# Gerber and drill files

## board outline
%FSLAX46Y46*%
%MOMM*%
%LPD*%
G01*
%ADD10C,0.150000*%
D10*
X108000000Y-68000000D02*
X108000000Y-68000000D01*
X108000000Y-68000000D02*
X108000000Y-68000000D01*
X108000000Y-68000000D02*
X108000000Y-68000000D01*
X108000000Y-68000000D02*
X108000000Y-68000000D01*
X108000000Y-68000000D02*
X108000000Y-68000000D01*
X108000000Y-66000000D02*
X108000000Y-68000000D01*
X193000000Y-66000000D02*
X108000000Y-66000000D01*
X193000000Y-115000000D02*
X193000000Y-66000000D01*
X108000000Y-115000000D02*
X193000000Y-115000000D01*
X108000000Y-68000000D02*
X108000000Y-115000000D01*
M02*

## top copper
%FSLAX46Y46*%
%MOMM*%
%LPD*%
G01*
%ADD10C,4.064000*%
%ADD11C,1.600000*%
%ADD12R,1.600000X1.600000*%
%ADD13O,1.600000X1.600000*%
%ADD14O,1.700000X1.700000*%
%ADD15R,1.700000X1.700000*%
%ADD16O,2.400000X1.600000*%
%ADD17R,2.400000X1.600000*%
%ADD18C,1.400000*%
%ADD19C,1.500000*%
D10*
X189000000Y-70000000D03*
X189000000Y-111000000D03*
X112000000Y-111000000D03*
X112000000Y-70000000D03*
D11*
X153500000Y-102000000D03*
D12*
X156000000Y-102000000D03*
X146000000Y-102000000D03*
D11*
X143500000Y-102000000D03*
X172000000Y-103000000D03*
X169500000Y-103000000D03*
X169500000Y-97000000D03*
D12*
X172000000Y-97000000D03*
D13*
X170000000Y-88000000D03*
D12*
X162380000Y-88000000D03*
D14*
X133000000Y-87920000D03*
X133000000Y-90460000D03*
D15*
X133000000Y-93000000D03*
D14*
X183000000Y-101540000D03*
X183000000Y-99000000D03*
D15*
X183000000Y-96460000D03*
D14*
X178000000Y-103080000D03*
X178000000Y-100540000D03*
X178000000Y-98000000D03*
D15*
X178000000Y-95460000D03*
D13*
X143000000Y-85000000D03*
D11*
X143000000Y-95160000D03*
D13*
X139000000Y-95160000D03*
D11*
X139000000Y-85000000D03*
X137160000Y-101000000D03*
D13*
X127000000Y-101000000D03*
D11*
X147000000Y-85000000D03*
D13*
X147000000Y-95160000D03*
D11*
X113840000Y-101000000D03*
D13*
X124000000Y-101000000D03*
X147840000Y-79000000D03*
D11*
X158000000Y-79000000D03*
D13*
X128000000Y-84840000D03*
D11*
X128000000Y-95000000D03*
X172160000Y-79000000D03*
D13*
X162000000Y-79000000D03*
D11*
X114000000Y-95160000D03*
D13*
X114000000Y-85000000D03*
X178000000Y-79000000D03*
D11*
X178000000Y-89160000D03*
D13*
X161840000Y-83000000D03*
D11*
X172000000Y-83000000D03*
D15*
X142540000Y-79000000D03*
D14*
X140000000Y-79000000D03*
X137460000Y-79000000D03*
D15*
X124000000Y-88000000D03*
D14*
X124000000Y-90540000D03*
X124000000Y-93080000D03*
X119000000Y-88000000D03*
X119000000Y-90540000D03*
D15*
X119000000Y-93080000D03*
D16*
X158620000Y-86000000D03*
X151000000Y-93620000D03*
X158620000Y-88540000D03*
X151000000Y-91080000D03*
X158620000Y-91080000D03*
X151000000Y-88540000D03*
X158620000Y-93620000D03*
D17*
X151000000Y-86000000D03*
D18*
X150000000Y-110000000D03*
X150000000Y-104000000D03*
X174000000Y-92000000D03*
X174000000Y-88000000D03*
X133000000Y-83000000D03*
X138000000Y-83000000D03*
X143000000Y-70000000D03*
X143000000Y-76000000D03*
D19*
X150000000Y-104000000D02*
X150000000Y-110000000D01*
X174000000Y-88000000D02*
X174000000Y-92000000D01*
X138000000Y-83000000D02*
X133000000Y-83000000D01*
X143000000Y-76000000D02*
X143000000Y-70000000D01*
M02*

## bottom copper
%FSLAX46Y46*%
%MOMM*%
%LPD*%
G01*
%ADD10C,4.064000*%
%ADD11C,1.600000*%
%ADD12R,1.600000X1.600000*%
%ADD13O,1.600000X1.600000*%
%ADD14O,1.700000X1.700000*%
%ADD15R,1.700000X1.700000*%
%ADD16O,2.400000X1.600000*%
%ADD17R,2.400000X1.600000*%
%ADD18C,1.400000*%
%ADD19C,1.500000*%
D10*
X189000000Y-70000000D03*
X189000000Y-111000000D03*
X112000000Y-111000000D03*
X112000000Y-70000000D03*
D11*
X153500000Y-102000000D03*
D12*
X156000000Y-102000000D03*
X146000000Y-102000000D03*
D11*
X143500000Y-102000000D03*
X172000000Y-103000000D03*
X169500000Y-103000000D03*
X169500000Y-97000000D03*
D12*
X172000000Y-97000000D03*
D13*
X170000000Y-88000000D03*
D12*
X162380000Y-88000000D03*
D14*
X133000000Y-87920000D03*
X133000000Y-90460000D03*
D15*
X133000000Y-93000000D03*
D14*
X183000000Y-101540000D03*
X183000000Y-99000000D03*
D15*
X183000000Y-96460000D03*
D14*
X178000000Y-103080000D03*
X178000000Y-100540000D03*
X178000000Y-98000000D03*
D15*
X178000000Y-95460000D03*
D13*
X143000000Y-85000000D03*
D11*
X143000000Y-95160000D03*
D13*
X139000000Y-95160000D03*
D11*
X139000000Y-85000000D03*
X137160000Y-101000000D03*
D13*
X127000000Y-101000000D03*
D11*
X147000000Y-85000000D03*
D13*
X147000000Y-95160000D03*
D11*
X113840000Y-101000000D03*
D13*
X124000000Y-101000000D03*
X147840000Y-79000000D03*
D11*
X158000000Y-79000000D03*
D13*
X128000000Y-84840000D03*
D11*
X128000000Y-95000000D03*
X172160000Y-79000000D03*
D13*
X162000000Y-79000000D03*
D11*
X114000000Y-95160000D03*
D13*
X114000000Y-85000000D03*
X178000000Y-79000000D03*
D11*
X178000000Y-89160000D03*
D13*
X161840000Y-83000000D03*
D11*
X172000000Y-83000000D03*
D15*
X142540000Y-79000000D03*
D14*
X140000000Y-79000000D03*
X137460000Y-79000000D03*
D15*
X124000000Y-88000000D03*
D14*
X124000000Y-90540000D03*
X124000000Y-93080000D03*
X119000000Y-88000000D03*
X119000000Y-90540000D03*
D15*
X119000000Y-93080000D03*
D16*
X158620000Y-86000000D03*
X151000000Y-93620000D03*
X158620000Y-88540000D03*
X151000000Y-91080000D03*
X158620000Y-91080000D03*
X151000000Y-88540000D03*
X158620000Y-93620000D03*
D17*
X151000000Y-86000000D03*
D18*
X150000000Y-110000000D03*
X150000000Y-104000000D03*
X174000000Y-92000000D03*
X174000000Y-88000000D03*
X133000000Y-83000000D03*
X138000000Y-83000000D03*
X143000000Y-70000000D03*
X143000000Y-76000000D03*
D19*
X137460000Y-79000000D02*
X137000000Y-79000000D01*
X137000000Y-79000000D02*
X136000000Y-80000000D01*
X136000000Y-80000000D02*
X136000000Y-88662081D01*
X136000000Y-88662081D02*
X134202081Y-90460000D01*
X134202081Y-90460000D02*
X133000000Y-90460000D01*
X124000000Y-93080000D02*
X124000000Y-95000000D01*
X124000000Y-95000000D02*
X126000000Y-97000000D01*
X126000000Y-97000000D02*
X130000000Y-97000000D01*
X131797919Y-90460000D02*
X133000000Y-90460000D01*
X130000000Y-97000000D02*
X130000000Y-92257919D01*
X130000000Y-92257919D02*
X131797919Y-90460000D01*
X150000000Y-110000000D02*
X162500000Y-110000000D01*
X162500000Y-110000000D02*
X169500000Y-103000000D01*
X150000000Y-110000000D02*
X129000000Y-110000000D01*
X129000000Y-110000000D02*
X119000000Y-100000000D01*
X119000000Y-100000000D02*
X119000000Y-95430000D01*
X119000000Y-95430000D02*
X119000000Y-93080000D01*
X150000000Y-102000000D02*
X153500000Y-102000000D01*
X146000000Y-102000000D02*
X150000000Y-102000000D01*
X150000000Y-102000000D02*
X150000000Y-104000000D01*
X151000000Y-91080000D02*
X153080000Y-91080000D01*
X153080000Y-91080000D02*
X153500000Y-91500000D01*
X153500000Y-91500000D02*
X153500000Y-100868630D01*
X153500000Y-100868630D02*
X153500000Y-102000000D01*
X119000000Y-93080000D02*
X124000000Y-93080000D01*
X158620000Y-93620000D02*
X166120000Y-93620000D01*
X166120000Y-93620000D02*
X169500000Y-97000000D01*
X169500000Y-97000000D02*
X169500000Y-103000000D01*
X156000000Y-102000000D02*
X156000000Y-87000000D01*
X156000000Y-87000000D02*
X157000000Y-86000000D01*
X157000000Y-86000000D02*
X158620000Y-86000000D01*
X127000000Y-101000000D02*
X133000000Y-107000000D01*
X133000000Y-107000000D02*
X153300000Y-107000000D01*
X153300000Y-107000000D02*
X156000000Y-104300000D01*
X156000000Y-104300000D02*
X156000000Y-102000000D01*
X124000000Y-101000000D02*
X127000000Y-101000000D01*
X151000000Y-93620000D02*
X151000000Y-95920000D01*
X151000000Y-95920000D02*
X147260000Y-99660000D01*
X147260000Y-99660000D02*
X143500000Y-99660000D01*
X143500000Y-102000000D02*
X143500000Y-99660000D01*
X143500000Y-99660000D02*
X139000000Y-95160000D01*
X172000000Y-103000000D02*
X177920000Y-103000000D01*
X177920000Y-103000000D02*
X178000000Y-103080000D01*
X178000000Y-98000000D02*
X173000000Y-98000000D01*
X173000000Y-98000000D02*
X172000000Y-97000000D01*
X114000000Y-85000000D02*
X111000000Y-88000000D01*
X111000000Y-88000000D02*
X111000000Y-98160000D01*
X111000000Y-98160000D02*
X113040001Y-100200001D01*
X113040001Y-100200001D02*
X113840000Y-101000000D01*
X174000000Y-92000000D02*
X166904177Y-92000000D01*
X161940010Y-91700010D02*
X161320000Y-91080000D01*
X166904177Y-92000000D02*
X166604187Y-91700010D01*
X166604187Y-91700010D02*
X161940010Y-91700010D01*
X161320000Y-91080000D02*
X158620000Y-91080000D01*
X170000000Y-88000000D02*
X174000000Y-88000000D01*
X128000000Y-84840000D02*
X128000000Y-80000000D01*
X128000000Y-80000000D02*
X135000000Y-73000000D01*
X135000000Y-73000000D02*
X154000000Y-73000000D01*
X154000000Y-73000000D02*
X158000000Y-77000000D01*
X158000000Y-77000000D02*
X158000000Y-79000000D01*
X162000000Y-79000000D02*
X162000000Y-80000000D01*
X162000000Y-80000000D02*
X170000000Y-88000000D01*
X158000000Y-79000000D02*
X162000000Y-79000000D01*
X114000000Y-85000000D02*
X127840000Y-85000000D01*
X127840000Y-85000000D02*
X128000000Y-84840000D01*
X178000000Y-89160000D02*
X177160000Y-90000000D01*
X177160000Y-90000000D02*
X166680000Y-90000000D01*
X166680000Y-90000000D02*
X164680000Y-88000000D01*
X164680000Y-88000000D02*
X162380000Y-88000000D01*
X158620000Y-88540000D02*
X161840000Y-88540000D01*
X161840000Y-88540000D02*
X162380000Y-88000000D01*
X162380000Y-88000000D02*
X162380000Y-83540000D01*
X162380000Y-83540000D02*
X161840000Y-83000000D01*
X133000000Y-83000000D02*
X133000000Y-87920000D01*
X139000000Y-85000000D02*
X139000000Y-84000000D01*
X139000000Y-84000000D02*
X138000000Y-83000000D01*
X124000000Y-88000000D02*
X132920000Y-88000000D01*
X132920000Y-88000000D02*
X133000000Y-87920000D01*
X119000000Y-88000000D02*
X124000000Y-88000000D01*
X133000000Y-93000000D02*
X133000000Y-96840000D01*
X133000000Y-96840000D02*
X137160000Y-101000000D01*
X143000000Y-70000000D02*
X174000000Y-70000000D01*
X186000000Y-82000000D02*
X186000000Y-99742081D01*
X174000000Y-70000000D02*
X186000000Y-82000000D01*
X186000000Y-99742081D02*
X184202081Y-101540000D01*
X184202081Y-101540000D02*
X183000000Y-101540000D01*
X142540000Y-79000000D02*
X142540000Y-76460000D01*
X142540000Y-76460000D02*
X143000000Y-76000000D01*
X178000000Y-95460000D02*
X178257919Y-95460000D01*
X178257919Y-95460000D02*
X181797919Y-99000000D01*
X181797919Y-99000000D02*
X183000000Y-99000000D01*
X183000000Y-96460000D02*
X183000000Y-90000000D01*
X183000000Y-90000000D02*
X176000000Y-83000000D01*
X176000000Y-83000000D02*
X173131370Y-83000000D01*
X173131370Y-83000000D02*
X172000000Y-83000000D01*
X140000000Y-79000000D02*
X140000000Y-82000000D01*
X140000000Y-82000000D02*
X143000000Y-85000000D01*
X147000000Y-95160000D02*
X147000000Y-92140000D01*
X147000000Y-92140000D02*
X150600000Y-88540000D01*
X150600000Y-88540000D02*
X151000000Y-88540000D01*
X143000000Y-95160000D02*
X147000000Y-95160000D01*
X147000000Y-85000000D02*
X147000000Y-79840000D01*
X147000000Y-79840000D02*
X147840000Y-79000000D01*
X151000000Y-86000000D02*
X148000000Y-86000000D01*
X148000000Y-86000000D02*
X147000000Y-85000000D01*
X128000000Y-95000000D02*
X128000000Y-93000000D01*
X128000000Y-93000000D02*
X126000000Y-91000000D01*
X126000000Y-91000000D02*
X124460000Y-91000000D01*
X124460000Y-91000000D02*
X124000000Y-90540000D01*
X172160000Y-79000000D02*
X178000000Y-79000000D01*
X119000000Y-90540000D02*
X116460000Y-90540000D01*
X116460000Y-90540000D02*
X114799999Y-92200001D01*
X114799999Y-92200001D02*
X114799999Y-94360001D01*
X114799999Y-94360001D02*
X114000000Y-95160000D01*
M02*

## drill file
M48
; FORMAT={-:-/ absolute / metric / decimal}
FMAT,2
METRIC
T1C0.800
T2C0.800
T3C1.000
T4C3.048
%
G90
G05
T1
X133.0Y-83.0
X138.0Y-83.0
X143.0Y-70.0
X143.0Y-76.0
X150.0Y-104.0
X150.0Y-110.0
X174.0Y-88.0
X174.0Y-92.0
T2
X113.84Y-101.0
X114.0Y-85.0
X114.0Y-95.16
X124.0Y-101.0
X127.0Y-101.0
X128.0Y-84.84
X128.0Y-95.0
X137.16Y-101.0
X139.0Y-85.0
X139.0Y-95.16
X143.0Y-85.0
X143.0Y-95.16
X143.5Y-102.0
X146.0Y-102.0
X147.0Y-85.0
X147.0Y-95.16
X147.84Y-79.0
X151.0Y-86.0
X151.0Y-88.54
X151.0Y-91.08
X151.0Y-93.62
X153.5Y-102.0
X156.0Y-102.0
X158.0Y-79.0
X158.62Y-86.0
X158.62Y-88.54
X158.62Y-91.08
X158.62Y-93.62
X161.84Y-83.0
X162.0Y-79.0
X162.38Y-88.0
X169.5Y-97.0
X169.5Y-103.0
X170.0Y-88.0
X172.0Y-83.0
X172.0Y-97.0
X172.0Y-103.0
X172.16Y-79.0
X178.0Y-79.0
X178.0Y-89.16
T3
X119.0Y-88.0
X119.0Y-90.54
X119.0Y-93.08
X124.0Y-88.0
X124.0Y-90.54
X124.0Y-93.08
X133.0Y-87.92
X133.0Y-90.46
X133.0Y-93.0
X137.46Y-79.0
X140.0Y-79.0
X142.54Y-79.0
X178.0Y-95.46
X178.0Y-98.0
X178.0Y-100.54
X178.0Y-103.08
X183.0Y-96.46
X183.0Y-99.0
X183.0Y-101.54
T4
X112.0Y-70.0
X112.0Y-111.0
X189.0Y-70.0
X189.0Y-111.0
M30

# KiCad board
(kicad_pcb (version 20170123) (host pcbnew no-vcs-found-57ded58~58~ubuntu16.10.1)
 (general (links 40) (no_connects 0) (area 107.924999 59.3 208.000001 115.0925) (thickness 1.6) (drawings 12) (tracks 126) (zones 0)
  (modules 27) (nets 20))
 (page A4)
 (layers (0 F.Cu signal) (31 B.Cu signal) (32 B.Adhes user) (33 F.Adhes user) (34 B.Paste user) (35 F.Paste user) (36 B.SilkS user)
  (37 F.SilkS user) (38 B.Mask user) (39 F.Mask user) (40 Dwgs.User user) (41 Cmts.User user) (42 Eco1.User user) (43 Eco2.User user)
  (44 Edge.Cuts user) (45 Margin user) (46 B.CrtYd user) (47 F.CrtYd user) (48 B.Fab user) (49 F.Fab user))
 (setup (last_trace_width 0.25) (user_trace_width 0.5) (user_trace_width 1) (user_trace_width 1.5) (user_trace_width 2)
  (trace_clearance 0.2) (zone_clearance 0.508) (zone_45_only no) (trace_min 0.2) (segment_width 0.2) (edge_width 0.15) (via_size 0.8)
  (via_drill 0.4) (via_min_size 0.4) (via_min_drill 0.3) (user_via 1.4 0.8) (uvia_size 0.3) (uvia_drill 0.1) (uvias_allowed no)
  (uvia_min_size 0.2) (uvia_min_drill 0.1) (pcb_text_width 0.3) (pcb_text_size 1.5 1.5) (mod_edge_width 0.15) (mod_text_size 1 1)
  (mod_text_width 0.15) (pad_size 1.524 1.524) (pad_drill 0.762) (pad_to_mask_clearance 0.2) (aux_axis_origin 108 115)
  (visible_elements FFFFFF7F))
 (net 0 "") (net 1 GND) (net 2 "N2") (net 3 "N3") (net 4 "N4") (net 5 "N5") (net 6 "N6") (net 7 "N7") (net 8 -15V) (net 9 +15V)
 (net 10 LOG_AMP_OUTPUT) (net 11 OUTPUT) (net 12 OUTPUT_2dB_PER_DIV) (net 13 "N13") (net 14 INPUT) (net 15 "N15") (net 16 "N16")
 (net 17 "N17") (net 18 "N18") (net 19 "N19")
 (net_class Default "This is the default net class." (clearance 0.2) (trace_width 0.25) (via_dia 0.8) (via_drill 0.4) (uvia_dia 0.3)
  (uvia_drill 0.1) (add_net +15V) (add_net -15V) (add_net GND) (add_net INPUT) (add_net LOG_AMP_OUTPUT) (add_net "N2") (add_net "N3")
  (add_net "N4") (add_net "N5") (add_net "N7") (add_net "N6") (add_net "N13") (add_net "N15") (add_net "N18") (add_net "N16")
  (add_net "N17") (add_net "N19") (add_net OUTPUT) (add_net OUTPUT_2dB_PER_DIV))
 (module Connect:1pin (layer F.Cu) (at 189 70)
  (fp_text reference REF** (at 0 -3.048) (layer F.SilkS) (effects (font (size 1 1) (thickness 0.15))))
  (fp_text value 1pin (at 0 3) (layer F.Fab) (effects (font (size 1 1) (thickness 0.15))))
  (pad 1 thru_hole circle (at 0 0) (size 4.064 4.064) (drill 3.048) (layers *.Cu *.Mask)))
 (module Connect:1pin (layer F.Cu) (at 189 111)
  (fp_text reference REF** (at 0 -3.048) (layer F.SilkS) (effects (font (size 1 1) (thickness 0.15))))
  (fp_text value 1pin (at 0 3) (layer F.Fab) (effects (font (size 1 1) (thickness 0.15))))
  (pad 1 thru_hole circle (at 0 0) (size 4.064 4.064) (drill 3.048) (layers *.Cu *.Mask)))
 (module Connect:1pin (layer F.Cu) (at 112 111)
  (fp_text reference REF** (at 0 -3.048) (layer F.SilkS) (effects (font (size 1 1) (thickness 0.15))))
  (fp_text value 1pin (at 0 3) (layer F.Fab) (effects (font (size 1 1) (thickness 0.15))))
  (pad 1 thru_hole circle (at 0 0) (size 4.064 4.064) (drill 3.048) (layers *.Cu *.Mask)))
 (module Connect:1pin (layer F.Cu) (at 112 70)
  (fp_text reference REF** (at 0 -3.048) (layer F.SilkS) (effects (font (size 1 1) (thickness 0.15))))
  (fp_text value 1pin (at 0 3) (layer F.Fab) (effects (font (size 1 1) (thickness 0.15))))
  (pad 1 thru_hole circle (at 0 0) (size 4.064 4.064) (drill 3.048) (layers *.Cu *.Mask)))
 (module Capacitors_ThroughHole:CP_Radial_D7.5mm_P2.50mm (layer F.Cu) (at 156 102 180)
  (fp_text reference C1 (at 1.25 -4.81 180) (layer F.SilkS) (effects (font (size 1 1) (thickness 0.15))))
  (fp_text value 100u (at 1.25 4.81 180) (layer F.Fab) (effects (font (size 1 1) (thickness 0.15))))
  (pad 2 thru_hole circle (at 2.5 0 180) (size 1.6 1.6) (drill 0.8) (layers *.Cu *.Mask) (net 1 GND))
  (pad 1 thru_hole rect (at 0 0 180) (size 1.6 1.6) (drill 0.8) (layers *.Cu *.Mask) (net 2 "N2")))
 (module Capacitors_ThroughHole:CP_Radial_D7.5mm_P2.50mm (layer F.Cu) (at 146 102 180)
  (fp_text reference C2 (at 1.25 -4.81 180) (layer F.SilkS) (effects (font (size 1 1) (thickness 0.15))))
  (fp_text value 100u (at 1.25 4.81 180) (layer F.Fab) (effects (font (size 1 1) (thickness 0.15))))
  (pad 1 thru_hole rect (at 0 0 180) (size 1.6 1.6) (drill 0.8) (layers *.Cu *.Mask) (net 1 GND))
  (pad 2 thru_hole circle (at 2.5 0 180) (size 1.6 1.6) (drill 0.8) (layers *.Cu *.Mask) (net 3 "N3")))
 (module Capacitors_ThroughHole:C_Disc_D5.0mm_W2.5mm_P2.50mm (layer F.Cu) (at 169.5 103)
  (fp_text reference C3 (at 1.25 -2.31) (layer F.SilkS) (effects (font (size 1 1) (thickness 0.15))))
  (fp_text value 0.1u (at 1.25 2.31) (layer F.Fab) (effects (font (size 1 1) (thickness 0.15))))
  (pad 2 thru_hole circle (at 2.5 0) (size 1.6 1.6) (drill 0.8) (layers *.Cu *.Mask) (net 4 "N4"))
  (pad 1 thru_hole circle (at 0 0) (size 1.6 1.6) (drill 0.8) (layers *.Cu *.Mask) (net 1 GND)))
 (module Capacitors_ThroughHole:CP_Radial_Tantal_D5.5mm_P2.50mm (layer F.Cu) (at 172 97 180)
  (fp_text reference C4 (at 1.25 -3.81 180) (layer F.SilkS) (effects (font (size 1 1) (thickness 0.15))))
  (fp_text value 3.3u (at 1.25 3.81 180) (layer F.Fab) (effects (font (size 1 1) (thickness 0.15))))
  (pad 2 thru_hole circle (at 2.5 0 180) (size 1.6 1.6) (drill 0.8) (layers *.Cu *.Mask) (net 1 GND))
  (pad 1 thru_hole rect (at 0 0 180) (size 1.6 1.6) (drill 0.8) (layers *.Cu *.Mask) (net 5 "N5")))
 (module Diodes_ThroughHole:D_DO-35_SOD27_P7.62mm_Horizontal (layer F.Cu) (at 162.38 88)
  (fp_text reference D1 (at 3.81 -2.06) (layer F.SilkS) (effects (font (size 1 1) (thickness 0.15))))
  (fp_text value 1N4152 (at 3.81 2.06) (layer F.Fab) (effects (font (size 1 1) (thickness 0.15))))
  (pad 2 thru_hole oval (at 7.62 0) (size 1.6 1.6) (drill 0.8) (layers *.Cu *.Mask) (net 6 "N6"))
  (pad 1 thru_hole rect (at 0 0) (size 1.6 1.6) (drill 0.8) (layers *.Cu *.Mask) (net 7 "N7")))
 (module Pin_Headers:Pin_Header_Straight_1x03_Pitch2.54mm (layer F.Cu) (at 133 93 180)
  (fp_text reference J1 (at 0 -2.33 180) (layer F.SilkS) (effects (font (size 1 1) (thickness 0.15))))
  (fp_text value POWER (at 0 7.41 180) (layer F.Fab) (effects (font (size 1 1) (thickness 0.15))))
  (pad 3 thru_hole oval (at 0 5.08 180) (size 1.7 1.7) (drill 1) (layers *.Cu *.Mask) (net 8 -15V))
  (pad 2 thru_hole oval (at 0 2.54 180) (size 1.7 1.7) (drill 1) (layers *.Cu *.Mask) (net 1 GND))
  (pad 1 thru_hole rect (at 0 0 180) (size 1.7 1.7) (drill 1) (layers *.Cu *.Mask) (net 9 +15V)))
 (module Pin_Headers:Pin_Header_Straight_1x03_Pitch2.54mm (layer F.Cu) (at 183 96.46)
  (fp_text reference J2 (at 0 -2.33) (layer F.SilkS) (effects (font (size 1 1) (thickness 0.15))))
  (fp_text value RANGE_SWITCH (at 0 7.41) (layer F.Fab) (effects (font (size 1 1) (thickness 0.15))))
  (pad 3 thru_hole oval (at 0 5.08) (size 1.7 1.7) (drill 1) (layers *.Cu *.Mask) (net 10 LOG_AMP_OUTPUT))
  (pad 2 thru_hole oval (at 0 2.54) (size 1.7 1.7) (drill 1) (layers *.Cu *.Mask) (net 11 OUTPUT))
  (pad 1 thru_hole rect (at 0 0) (size 1.7 1.7) (drill 1) (layers *.Cu *.Mask) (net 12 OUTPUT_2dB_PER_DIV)))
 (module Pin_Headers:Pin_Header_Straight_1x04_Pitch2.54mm (layer F.Cu) (at 178 95.46)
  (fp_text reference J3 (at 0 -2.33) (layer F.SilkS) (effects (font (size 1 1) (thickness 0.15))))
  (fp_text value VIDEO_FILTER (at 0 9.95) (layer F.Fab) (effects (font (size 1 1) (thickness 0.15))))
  (pad 4 thru_hole oval (at 0 7.62) (size 1.7 1.7) (drill 1) (layers *.Cu *.Mask) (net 4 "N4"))
  (pad 3 thru_hole oval (at 0 5.08) (size 1.7 1.7) (drill 1) (layers *.Cu *.Mask) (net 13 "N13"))
  (pad 2 thru_hole oval (at 0 2.54) (size 1.7 1.7) (drill 1) (layers *.Cu *.Mask) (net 5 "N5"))
  (pad 1 thru_hole rect (at 0 0) (size 1.7 1.7) (drill 1) (layers *.Cu *.Mask) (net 11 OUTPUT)))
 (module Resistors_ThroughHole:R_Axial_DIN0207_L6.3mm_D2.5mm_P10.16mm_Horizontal (layer F.Cu) (at 143 95.16 90)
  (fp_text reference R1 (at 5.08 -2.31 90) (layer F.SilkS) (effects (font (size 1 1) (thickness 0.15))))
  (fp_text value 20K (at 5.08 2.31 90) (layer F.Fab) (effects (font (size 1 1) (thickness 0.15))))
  (pad 2 thru_hole oval (at 10.16 0 90) (size 1.6 1.6) (drill 0.8) (layers *.Cu *.Mask) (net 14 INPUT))
  (pad 1 thru_hole circle (at 0 0 90) (size 1.6 1.6) (drill 0.8) (layers *.Cu *.Mask) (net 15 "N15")))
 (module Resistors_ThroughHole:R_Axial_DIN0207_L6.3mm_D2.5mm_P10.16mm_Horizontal (layer F.Cu) (at 139 85 270)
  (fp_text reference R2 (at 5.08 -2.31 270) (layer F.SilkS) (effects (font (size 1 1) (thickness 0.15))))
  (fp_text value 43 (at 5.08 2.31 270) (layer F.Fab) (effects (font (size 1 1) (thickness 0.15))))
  (pad 2 thru_hole oval (at 10.16 0 270) (size 1.6 1.6) (drill 0.8) (layers *.Cu *.Mask) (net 3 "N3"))
  (pad 1 thru_hole circle (at 0 0 270) (size 1.6 1.6) (drill 0.8) (layers *.Cu *.Mask) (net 8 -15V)))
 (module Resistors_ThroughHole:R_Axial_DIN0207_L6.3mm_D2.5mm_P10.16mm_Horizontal (layer F.Cu) (at 137.16 101 180)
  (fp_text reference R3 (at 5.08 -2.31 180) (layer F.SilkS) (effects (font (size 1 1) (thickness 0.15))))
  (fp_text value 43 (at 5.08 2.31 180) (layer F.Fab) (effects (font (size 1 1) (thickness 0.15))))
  (pad 1 thru_hole circle (at 0 0 180) (size 1.6 1.6) (drill 0.8) (layers *.Cu *.Mask) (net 9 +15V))
  (pad 2 thru_hole oval (at 10.16 0 180) (size 1.6 1.6) (drill 0.8) (layers *.Cu *.Mask) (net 2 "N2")))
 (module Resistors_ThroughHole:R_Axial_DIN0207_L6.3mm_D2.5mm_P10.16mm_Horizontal (layer F.Cu) (at 147 85 270)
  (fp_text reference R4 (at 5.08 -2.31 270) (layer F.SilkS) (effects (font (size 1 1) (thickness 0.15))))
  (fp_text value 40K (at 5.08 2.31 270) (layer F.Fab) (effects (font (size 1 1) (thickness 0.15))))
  (pad 1 thru_hole circle (at 0 0 270) (size 1.6 1.6) (drill 0.8) (layers *.Cu *.Mask) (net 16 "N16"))
  (pad 2 thru_hole oval (at 10.16 0 270) (size 1.6 1.6) (drill 0.8) (layers *.Cu *.Mask) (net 15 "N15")))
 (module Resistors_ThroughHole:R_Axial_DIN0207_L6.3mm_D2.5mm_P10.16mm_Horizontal (layer F.Cu) (at 113.84 101)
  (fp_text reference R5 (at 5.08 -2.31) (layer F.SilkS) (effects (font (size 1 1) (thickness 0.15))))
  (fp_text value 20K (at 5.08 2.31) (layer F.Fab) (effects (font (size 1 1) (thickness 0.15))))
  (pad 1 thru_hole circle (at 0 0) (size 1.6 1.6) (drill 0.8) (layers *.Cu *.Mask) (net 6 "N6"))
  (pad 2 thru_hole oval (at 10.16 0) (size 1.6 1.6) (drill 0.8) (layers *.Cu *.Mask) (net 2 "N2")))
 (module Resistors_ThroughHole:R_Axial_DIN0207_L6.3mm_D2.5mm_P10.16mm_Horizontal (layer F.Cu) (at 158 79 180)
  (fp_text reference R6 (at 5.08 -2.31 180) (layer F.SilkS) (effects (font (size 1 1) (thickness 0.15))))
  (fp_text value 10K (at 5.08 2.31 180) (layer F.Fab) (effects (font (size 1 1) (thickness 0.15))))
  (pad 2 thru_hole oval (at 10.16 0 180) (size 1.6 1.6) (drill 0.8) (layers *.Cu *.Mask) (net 16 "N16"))
  (pad 1 thru_hole circle (at 0 0 180) (size 1.6 1.6) (drill 0.8) (layers *.Cu *.Mask) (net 6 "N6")))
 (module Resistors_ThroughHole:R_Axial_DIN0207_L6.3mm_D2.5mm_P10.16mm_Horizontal (layer F.Cu) (at 128 95 90)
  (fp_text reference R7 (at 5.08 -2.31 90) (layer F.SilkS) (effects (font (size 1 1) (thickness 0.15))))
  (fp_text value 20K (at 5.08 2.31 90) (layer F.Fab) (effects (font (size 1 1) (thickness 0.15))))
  (pad 2 thru_hole oval (at 10.16 0 90) (size 1.6 1.6) (drill 0.8) (layers *.Cu *.Mask) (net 6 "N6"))
  (pad 1 thru_hole circle (at 0 0 90) (size 1.6 1.6) (drill 0.8) (layers *.Cu *.Mask) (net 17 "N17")))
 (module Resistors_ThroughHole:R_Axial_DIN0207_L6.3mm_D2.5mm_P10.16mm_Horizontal (layer F.Cu) (at 172.16 79 180)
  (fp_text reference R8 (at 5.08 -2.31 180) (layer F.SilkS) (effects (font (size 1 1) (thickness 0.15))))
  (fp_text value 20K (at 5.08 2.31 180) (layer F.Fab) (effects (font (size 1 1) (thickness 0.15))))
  (pad 1 thru_hole circle (at 0 0 180) (size 1.6 1.6) (drill 0.8) (layers *.Cu *.Mask) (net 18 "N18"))
  (pad 2 thru_hole oval (at 10.16 0 180) (size 1.6 1.6) (drill 0.8) (layers *.Cu *.Mask) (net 6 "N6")))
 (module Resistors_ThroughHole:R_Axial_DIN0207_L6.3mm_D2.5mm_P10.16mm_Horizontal (layer F.Cu) (at 114 95.16 90)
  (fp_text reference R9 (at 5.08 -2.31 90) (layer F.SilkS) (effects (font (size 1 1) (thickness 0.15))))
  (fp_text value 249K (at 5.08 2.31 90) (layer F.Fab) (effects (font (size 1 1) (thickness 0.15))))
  (pad 1 thru_hole circle (at 0 0 90) (size 1.6 1.6) (drill 0.8) (layers *.Cu *.Mask) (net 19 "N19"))
  (pad 2 thru_hole oval (at 10.16 0 90) (size 1.6 1.6) (drill 0.8) (layers *.Cu *.Mask) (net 6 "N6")))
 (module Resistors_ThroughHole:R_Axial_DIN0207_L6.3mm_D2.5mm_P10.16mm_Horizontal (layer F.Cu) (at 178 89.16 90)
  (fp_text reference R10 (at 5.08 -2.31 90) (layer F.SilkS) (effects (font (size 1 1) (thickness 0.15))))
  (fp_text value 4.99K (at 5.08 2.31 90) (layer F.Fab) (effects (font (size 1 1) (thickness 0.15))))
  (pad 2 thru_hole oval (at 10.16 0 90) (size 1.6 1.6) (drill 0.8) (layers *.Cu *.Mask) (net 18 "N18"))
  (pad 1 thru_hole circle (at 0 0 90) (size 1.6 1.6) (drill 0.8) (layers *.Cu *.Mask) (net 7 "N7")))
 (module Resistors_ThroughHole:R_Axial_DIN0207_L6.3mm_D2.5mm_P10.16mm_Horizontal (layer F.Cu) (at 172 83 180)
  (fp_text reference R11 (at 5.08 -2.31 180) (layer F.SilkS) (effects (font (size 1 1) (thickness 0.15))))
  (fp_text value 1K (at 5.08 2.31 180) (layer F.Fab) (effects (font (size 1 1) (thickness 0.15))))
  (pad 2 thru_hole oval (at 10.16 0 180) (size 1.6 1.6) (drill 0.8) (layers *.Cu *.Mask) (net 7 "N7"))
  (pad 1 thru_hole circle (at 0 0 180) (size 1.6 1.6) (drill 0.8) (layers *.Cu *.Mask) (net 12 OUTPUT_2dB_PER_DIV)))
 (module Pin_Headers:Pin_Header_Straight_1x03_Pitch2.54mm (layer F.Cu) (at 142.54 79 270)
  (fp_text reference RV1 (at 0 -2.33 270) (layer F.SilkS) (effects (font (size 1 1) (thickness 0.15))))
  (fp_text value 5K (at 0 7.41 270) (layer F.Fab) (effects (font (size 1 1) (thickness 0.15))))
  (pad 1 thru_hole rect (at 0 0 270) (size 1.7 1.7) (drill 1) (layers *.Cu *.Mask) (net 10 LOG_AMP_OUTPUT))
  (pad 2 thru_hole oval (at 0 2.54 270) (size 1.7 1.7) (drill 1) (layers *.Cu *.Mask) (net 14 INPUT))
  (pad 3 thru_hole oval (at 0 5.08 270) (size 1.7 1.7) (drill 1) (layers *.Cu *.Mask) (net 1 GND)))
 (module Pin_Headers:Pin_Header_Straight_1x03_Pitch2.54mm (layer F.Cu) (at 124 88)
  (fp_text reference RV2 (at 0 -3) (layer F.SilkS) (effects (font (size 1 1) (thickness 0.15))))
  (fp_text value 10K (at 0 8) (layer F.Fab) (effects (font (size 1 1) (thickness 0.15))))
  (pad 1 thru_hole rect (at 0 0) (size 1.7 1.7) (drill 1) (layers *.Cu *.Mask) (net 8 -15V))
  (pad 2 thru_hole oval (at 0 2.54) (size 1.7 1.7) (drill 1) (layers *.Cu *.Mask) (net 17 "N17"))
  (pad 3 thru_hole oval (at 0 5.08) (size 1.7 1.7) (drill 1) (layers *.Cu *.Mask) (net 1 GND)))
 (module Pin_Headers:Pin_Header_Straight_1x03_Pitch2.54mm (layer F.Cu) (at 119 93.08 180)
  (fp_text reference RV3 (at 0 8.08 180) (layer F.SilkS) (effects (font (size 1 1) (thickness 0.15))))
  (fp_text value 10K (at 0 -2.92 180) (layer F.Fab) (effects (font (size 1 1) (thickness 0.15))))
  (pad 3 thru_hole oval (at 0 5.08 180) (size 1.7 1.7) (drill 1) (layers *.Cu *.Mask) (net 8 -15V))
  (pad 2 thru_hole oval (at 0 2.54 180) (size 1.7 1.7) (drill 1) (layers *.Cu *.Mask) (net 19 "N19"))
  (pad 1 thru_hole rect (at 0 0 180) (size 1.7 1.7) (drill 1) (layers *.Cu *.Mask) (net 1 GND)))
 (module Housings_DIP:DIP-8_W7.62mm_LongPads (layer F.Cu) (at 151 86)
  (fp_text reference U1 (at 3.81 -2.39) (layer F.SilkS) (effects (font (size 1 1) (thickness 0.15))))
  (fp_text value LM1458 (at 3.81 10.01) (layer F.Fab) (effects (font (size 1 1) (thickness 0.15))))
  (pad 8 thru_hole oval (at 7.62 0) (size 2.4 1.6) (drill 0.8) (layers *.Cu *.Mask) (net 2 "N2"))
  (pad 4 thru_hole oval (at 0 7.62) (size 2.4 1.6) (drill 0.8) (layers *.Cu *.Mask) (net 3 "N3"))
  (pad 7 thru_hole oval (at 7.62 2.54) (size 2.4 1.6) (drill 0.8) (layers *.Cu *.Mask) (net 7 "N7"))
  (pad 3 thru_hole oval (at 0 5.08) (size 2.4 1.6) (drill 0.8) (layers *.Cu *.Mask) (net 1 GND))
  (pad 6 thru_hole oval (at 7.62 5.08) (size 2.4 1.6) (drill 0.8) (layers *.Cu *.Mask) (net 6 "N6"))
  (pad 2 thru_hole oval (at 0 2.54) (size 2.4 1.6) (drill 0.8) (layers *.Cu *.Mask) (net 15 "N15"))
  (pad 5 thru_hole oval (at 7.62 7.62) (size 2.4 1.6) (drill 0.8) (layers *.Cu *.Mask) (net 1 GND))
  (pad 1 thru_hole rect (at 0 0) (size 2.4 1.6) (drill 0.8) (layers *.Cu *.Mask) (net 16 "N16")))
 (gr_line (start 108 68) (end 108 68) (layer Edge.Cuts) (width 0.15))
 (gr_line (start 108 68) (end 108 68) (layer Edge.Cuts) (width 0.15))
 (gr_line (start 108 68) (end 108 68) (layer Edge.Cuts) (width 0.15))
 (gr_line (start 108 68) (end 108 68) (layer Edge.Cuts) (width 0.15))
 (gr_line (start 108 68) (end 108 68) (layer Edge.Cuts) (width 0.15))
 (gr_line (start 108 66) (end 108 68) (layer Edge.Cuts) (width 0.15))
 (gr_line (start 193 66) (end 108 66) (layer Edge.Cuts) (width 0.15))
 (gr_line (start 193 115) (end 193 66) (layer Edge.Cuts) (width 0.15))
 (gr_line (start 108 115) (end 193 115) (layer Edge.Cuts) (width 0.15))
 (gr_line (start 108 68) (end 108 115) (layer Edge.Cuts) (width 0.15))
 (segment (start 137.46 79) (end 137 79) (width 1.5) (layer B.Cu) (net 1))
 (segment (start 137 79) (end 136 80) (width 1.5) (layer B.Cu) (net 1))
 (segment (start 136 80) (end 136 88.662081) (width 1.5) (layer B.Cu) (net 1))
 (segment (start 136 88.662081) (end 134.202081 90.46) (width 1.5) (layer B.Cu) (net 1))
 (segment (start 134.202081 90.46) (end 133 90.46) (width 1.5) (layer B.Cu) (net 1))
 (segment (start 124 93.08) (end 124 95) (width 1.5) (layer B.Cu) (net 1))
 (segment (start 124 95) (end 126 97) (width 1.5) (layer B.Cu) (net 1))
 (segment (start 126 97) (end 130 97) (width 1.5) (layer B.Cu) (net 1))
 (segment (start 131.797919 90.46) (end 133 90.46) (width 1.5) (layer B.Cu) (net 1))
 (segment (start 130 97) (end 130 92.257919) (width 1.5) (layer B.Cu) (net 1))
 (segment (start 130 92.257919) (end 131.797919 90.46) (width 1.5) (layer B.Cu) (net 1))
 (segment (start 150 110) (end 162.5 110) (width 1.5) (layer B.Cu) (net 1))
 (segment (start 162.5 110) (end 169.5 103) (width 1.5) (layer B.Cu) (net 1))
 (segment (start 150 110) (end 129 110) (width 1.5) (layer B.Cu) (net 1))
 (segment (start 129 110) (end 119 100) (width 1.5) (layer B.Cu) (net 1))
 (segment (start 119 100) (end 119 95.43) (width 1.5) (layer B.Cu) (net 1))
 (segment (start 119 95.43) (end 119 93.08) (width 1.5) (layer B.Cu) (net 1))
 (segment (start 150 104) (end 150 110) (width 1.5) (layer F.Cu) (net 1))
 (via (at 150 110) (size 1.4) (drill 0.8) (layers F.Cu B.Cu) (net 1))
 (segment (start 150 102) (end 153.5 102) (width 1.5) (layer B.Cu) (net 1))
 (segment (start 146 102) (end 150 102) (width 1.5) (layer B.Cu) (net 1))
 (segment (start 150 102) (end 150 104) (width 1.5) (layer B.Cu) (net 1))
 (via (at 150 104) (size 1.4) (drill 0.8) (layers F.Cu B.Cu) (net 1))
 (segment (start 151 91.08) (end 153.08 91.08) (width 1.5) (layer B.Cu) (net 1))
 (segment (start 153.08 91.08) (end 153.5 91.5) (width 1.5) (layer B.Cu) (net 1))
 (segment (start 153.5 91.5) (end 153.5 100.86863) (width 1.5) (layer B.Cu) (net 1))
 (segment (start 153.5 100.86863) (end 153.5 102) (width 1.5) (layer B.Cu) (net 1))
 (segment (start 119 93.08) (end 124 93.08) (width 1.5) (layer B.Cu) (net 1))
 (segment (start 158.62 93.62) (end 166.12 93.62) (width 1.5) (layer B.Cu) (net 1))
 (segment (start 166.12 93.62) (end 169.5 97) (width 1.5) (layer B.Cu) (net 1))
 (segment (start 169.5 97) (end 169.5 103) (width 1.5) (layer B.Cu) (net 1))
 (segment (start 156 102) (end 156 87) (width 1.5) (layer B.Cu) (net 2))
 (segment (start 156 87) (end 157 86) (width 1.5) (layer B.Cu) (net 2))
 (segment (start 157 86) (end 158.62 86) (width 1.5) (layer B.Cu) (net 2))
 (segment (start 127 101) (end 133 107) (width 1.5) (layer B.Cu) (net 2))
 (segment (start 133 107) (end 153.3 107) (width 1.5) (layer B.Cu) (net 2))
 (segment (start 153.3 107) (end 156 104.3) (width 1.5) (layer B.Cu) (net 2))
 (segment (start 156 104.3) (end 156 102) (width 1.5) (layer B.Cu) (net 2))
 (segment (start 124 101) (end 127 101) (width 1.5) (layer B.Cu) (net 2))
 (segment (start 151 93.62) (end 151 95.92) (width 1.5) (layer B.Cu) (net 3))
 (segment (start 151 95.92) (end 147.26 99.66) (width 1.5) (layer B.Cu) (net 3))
 (segment (start 147.26 99.66) (end 143.5 99.66) (width 1.5) (layer B.Cu) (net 3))
 (segment (start 143.5 102) (end 143.5 99.66) (width 1.5) (layer B.Cu) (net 3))
 (segment (start 143.5 99.66) (end 139 95.16) (width 1.5) (layer B.Cu) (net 3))
 (segment (start 172 103) (end 177.92 103) (width 1.5) (layer B.Cu) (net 4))
 (segment (start 177.92 103) (end 178 103.08) (width 1.5) (layer B.Cu) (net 4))
 (segment (start 178 98) (end 173 98) (width 1.5) (layer B.Cu) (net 5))
 (segment (start 173 98) (end 172 97) (width 1.5) (layer B.Cu) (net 5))
 (segment (start 114 85) (end 111 88) (width 1.5) (layer B.Cu) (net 6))
 (segment (start 111 88) (end 111 98.16) (width 1.5) (layer B.Cu) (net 6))
 (segment (start 111 98.16) (end 113.040001 100.200001) (width 1.5) (layer B.Cu) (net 6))
 (segment (start 113.040001 100.200001) (end 113.84 101) (width 1.5) (layer B.Cu) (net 6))
 (segment (start 174 92) (end 166.904177 92) (width 1.5) (layer B.Cu) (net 6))
 (segment (start 161.94001 91.70001) (end 161.32 91.08) (width 1.5) (layer B.Cu) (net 6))
 (segment (start 166.904177 92) (end 166.604187 91.70001) (width 1.5) (layer B.Cu) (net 6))
 (segment (start 166.604187 91.70001) (end 161.94001 91.70001) (width 1.5) (layer B.Cu) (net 6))
 (segment (start 161.32 91.08) (end 158.62 91.08) (width 1.5) (layer B.Cu) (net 6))
 (segment (start 174 88) (end 174 92) (width 1.5) (layer F.Cu) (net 6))
 (via (at 174 92) (size 1.4) (drill 0.8) (layers F.Cu B.Cu) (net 6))
 (segment (start 170 88) (end 174 88) (width 1.5) (layer B.Cu) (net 6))
 (via (at 174 88) (size 1.4) (drill 0.8) (layers F.Cu B.Cu) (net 6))
 (segment (start 128 84.84) (end 128 80) (width 1.5) (layer B.Cu) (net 6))
 (segment (start 128 80) (end 135 73) (width 1.5) (layer B.Cu) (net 6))
 (segment (start 135 73) (end 154 73) (width 1.5) (layer B.Cu) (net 6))
 (segment (start 154 73) (end 158 77) (width 1.5) (layer B.Cu) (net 6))
 (segment (start 158 77) (end 158 79) (width 1.5) (layer B.Cu) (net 6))
 (segment (start 162 79) (end 162 80) (width 1.5) (layer B.Cu) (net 6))
 (segment (start 162 80) (end 170 88) (width 1.5) (layer B.Cu) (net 6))
 (segment (start 158 79) (end 162 79) (width 1.5) (layer B.Cu) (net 6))
 (segment (start 114 85) (end 127.84 85) (width 1.5) (layer B.Cu) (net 6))
 (segment (start 127.84 85) (end 128 84.84) (width 1.5) (layer B.Cu) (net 6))
 (segment (start 178 89.16) (end 177.16 90) (width 1.5) (layer B.Cu) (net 7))
 (segment (start 177.16 90) (end 166.68 90) (width 1.5) (layer B.Cu) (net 7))
 (segment (start 166.68 90) (end 164.68 88) (width 1.5) (layer B.Cu) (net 7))
 (segment (start 164.68 88) (end 162.38 88) (width 1.5) (layer B.Cu) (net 7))
 (segment (start 158.62 88.54) (end 161.84 88.54) (width 1.5) (layer B.Cu) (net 7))
 (segment (start 161.84 88.54) (end 162.38 88) (width 1.5) (layer B.Cu) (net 7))
 (segment (start 162.38 88) (end 162.38 83.54) (width 1.5) (layer B.Cu) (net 7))
 (segment (start 162.38 83.54) (end 161.84 83) (width 1.5) (layer B.Cu) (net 7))
 (segment (start 133 83) (end 133 87.92) (width 1.5) (layer B.Cu) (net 8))
 (segment (start 138 83) (end 133 83) (width 1.5) (layer F.Cu) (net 8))
 (via (at 133 83) (size 1.4) (drill 0.8) (layers F.Cu B.Cu) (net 8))
 (segment (start 139 85) (end 139 84) (width 1.5) (layer B.Cu) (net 8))
 (segment (start 139 84) (end 138 83) (width 1.5) (layer B.Cu) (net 8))
 (via (at 138 83) (size 1.4) (drill 0.8) (layers F.Cu B.Cu) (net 8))
 (segment (start 124 88) (end 132.92 88) (width 1.5) (layer B.Cu) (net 8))
 (segment (start 132.92 88) (end 133 87.92) (width 1.5) (layer B.Cu) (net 8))
 (segment (start 119 88) (end 124 88) (width 1.5) (layer B.Cu) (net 8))
 (segment (start 133 93) (end 133 96.84) (width 1.5) (layer B.Cu) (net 9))
 (segment (start 133 96.84) (end 137.16 101) (width 1.5) (layer B.Cu) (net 9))
 (segment (start 143 70) (end 174 70) (width 1.5) (layer B.Cu) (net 10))
 (segment (start 186 82) (end 186 99.742081) (width 1.5) (layer B.Cu) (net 10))
 (segment (start 174 70) (end 186 82) (width 1.5) (layer B.Cu) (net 10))
 (segment (start 186 99.742081) (end 184.202081 101.54) (width 1.5) (layer B.Cu) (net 10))
 (segment (start 184.202081 101.54) (end 183 101.54) (width 1.5) (layer B.Cu) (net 10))
 (segment (start 143 76) (end 143 70) (width 1.5) (layer F.Cu) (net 10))
 (via (at 143 70) (size 1.4) (drill 0.8) (layers F.Cu B.Cu) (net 10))
 (segment (start 142.54 79) (end 142.54 76.46) (width 1.5) (layer B.Cu) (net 10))
 (segment (start 142.54 76.46) (end 143 76) (width 1.5) (layer B.Cu) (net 10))
 (via (at 143 76) (size 1.4) (drill 0.8) (layers F.Cu B.Cu) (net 10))
 (segment (start 178 95.46) (end 178.257919 95.46) (width 1.5) (layer B.Cu) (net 11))
 (segment (start 178.257919 95.46) (end 181.797919 99) (width 1.5) (layer B.Cu) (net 11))
 (segment (start 181.797919 99) (end 183 99) (width 1.5) (layer B.Cu) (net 11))
 (segment (start 183 96.46) (end 183 90) (width 1.5) (layer B.Cu) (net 12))
 (segment (start 183 90) (end 176 83) (width 1.5) (layer B.Cu) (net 12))
 (segment (start 176 83) (end 173.13137 83) (width 1.5) (layer B.Cu) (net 12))
 (segment (start 173.13137 83) (end 172 83) (width 1.5) (layer B.Cu) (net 12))
 (segment (start 140 79) (end 140 82) (width 1.5) (layer B.Cu) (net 14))
 (segment (start 140 82) (end 143 85) (width 1.5) (layer B.Cu) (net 14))
 (segment (start 147 95.16) (end 147 92.14) (width 1.5) (layer B.Cu) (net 15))
 (segment (start 147 92.14) (end 150.6 88.54) (width 1.5) (layer B.Cu) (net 15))
 (segment (start 150.6 88.54) (end 151 88.54) (width 1.5) (layer B.Cu) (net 15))
 (segment (start 143 95.16) (end 147 95.16) (width 1.5) (layer B.Cu) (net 15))
 (segment (start 147 85) (end 147 79.84) (width 1.5) (layer B.Cu) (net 16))
 (segment (start 147 79.84) (end 147.84 79) (width 1.5) (layer B.Cu) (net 16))
 (segment (start 151 86) (end 148 86) (width 1.5) (layer B.Cu) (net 16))
 (segment (start 148 86) (end 147 85) (width 1.5) (layer B.Cu) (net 16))
 (segment (start 128 95) (end 128 93) (width 1.5) (layer B.Cu) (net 17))
 (segment (start 128 93) (end 126 91) (width 1.5) (layer B.Cu) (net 17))
 (segment (start 126 91) (end 124.46 91) (width 1.5) (layer B.Cu) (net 17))
 (segment (start 124.46 91) (end 124 90.54) (width 1.5) (layer B.Cu) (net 17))
 (segment (start 172.16 79) (end 178 79) (width 1.5) (layer B.Cu) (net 18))
 (segment (start 119 90.54) (end 116.46 90.54) (width 1.5) (layer B.Cu) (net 19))
 (segment (start 116.46 90.54) (end 114.799999 92.200001) (width 1.5) (layer B.Cu) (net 19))
 (segment (start 114.799999 92.200001) (end 114.799999 94.360001) (width 1.5) (layer B.Cu) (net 19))
 (segment (start 114.799999 94.360001) (end 114 95.16) (width 1.5) (layer B.Cu) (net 19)))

